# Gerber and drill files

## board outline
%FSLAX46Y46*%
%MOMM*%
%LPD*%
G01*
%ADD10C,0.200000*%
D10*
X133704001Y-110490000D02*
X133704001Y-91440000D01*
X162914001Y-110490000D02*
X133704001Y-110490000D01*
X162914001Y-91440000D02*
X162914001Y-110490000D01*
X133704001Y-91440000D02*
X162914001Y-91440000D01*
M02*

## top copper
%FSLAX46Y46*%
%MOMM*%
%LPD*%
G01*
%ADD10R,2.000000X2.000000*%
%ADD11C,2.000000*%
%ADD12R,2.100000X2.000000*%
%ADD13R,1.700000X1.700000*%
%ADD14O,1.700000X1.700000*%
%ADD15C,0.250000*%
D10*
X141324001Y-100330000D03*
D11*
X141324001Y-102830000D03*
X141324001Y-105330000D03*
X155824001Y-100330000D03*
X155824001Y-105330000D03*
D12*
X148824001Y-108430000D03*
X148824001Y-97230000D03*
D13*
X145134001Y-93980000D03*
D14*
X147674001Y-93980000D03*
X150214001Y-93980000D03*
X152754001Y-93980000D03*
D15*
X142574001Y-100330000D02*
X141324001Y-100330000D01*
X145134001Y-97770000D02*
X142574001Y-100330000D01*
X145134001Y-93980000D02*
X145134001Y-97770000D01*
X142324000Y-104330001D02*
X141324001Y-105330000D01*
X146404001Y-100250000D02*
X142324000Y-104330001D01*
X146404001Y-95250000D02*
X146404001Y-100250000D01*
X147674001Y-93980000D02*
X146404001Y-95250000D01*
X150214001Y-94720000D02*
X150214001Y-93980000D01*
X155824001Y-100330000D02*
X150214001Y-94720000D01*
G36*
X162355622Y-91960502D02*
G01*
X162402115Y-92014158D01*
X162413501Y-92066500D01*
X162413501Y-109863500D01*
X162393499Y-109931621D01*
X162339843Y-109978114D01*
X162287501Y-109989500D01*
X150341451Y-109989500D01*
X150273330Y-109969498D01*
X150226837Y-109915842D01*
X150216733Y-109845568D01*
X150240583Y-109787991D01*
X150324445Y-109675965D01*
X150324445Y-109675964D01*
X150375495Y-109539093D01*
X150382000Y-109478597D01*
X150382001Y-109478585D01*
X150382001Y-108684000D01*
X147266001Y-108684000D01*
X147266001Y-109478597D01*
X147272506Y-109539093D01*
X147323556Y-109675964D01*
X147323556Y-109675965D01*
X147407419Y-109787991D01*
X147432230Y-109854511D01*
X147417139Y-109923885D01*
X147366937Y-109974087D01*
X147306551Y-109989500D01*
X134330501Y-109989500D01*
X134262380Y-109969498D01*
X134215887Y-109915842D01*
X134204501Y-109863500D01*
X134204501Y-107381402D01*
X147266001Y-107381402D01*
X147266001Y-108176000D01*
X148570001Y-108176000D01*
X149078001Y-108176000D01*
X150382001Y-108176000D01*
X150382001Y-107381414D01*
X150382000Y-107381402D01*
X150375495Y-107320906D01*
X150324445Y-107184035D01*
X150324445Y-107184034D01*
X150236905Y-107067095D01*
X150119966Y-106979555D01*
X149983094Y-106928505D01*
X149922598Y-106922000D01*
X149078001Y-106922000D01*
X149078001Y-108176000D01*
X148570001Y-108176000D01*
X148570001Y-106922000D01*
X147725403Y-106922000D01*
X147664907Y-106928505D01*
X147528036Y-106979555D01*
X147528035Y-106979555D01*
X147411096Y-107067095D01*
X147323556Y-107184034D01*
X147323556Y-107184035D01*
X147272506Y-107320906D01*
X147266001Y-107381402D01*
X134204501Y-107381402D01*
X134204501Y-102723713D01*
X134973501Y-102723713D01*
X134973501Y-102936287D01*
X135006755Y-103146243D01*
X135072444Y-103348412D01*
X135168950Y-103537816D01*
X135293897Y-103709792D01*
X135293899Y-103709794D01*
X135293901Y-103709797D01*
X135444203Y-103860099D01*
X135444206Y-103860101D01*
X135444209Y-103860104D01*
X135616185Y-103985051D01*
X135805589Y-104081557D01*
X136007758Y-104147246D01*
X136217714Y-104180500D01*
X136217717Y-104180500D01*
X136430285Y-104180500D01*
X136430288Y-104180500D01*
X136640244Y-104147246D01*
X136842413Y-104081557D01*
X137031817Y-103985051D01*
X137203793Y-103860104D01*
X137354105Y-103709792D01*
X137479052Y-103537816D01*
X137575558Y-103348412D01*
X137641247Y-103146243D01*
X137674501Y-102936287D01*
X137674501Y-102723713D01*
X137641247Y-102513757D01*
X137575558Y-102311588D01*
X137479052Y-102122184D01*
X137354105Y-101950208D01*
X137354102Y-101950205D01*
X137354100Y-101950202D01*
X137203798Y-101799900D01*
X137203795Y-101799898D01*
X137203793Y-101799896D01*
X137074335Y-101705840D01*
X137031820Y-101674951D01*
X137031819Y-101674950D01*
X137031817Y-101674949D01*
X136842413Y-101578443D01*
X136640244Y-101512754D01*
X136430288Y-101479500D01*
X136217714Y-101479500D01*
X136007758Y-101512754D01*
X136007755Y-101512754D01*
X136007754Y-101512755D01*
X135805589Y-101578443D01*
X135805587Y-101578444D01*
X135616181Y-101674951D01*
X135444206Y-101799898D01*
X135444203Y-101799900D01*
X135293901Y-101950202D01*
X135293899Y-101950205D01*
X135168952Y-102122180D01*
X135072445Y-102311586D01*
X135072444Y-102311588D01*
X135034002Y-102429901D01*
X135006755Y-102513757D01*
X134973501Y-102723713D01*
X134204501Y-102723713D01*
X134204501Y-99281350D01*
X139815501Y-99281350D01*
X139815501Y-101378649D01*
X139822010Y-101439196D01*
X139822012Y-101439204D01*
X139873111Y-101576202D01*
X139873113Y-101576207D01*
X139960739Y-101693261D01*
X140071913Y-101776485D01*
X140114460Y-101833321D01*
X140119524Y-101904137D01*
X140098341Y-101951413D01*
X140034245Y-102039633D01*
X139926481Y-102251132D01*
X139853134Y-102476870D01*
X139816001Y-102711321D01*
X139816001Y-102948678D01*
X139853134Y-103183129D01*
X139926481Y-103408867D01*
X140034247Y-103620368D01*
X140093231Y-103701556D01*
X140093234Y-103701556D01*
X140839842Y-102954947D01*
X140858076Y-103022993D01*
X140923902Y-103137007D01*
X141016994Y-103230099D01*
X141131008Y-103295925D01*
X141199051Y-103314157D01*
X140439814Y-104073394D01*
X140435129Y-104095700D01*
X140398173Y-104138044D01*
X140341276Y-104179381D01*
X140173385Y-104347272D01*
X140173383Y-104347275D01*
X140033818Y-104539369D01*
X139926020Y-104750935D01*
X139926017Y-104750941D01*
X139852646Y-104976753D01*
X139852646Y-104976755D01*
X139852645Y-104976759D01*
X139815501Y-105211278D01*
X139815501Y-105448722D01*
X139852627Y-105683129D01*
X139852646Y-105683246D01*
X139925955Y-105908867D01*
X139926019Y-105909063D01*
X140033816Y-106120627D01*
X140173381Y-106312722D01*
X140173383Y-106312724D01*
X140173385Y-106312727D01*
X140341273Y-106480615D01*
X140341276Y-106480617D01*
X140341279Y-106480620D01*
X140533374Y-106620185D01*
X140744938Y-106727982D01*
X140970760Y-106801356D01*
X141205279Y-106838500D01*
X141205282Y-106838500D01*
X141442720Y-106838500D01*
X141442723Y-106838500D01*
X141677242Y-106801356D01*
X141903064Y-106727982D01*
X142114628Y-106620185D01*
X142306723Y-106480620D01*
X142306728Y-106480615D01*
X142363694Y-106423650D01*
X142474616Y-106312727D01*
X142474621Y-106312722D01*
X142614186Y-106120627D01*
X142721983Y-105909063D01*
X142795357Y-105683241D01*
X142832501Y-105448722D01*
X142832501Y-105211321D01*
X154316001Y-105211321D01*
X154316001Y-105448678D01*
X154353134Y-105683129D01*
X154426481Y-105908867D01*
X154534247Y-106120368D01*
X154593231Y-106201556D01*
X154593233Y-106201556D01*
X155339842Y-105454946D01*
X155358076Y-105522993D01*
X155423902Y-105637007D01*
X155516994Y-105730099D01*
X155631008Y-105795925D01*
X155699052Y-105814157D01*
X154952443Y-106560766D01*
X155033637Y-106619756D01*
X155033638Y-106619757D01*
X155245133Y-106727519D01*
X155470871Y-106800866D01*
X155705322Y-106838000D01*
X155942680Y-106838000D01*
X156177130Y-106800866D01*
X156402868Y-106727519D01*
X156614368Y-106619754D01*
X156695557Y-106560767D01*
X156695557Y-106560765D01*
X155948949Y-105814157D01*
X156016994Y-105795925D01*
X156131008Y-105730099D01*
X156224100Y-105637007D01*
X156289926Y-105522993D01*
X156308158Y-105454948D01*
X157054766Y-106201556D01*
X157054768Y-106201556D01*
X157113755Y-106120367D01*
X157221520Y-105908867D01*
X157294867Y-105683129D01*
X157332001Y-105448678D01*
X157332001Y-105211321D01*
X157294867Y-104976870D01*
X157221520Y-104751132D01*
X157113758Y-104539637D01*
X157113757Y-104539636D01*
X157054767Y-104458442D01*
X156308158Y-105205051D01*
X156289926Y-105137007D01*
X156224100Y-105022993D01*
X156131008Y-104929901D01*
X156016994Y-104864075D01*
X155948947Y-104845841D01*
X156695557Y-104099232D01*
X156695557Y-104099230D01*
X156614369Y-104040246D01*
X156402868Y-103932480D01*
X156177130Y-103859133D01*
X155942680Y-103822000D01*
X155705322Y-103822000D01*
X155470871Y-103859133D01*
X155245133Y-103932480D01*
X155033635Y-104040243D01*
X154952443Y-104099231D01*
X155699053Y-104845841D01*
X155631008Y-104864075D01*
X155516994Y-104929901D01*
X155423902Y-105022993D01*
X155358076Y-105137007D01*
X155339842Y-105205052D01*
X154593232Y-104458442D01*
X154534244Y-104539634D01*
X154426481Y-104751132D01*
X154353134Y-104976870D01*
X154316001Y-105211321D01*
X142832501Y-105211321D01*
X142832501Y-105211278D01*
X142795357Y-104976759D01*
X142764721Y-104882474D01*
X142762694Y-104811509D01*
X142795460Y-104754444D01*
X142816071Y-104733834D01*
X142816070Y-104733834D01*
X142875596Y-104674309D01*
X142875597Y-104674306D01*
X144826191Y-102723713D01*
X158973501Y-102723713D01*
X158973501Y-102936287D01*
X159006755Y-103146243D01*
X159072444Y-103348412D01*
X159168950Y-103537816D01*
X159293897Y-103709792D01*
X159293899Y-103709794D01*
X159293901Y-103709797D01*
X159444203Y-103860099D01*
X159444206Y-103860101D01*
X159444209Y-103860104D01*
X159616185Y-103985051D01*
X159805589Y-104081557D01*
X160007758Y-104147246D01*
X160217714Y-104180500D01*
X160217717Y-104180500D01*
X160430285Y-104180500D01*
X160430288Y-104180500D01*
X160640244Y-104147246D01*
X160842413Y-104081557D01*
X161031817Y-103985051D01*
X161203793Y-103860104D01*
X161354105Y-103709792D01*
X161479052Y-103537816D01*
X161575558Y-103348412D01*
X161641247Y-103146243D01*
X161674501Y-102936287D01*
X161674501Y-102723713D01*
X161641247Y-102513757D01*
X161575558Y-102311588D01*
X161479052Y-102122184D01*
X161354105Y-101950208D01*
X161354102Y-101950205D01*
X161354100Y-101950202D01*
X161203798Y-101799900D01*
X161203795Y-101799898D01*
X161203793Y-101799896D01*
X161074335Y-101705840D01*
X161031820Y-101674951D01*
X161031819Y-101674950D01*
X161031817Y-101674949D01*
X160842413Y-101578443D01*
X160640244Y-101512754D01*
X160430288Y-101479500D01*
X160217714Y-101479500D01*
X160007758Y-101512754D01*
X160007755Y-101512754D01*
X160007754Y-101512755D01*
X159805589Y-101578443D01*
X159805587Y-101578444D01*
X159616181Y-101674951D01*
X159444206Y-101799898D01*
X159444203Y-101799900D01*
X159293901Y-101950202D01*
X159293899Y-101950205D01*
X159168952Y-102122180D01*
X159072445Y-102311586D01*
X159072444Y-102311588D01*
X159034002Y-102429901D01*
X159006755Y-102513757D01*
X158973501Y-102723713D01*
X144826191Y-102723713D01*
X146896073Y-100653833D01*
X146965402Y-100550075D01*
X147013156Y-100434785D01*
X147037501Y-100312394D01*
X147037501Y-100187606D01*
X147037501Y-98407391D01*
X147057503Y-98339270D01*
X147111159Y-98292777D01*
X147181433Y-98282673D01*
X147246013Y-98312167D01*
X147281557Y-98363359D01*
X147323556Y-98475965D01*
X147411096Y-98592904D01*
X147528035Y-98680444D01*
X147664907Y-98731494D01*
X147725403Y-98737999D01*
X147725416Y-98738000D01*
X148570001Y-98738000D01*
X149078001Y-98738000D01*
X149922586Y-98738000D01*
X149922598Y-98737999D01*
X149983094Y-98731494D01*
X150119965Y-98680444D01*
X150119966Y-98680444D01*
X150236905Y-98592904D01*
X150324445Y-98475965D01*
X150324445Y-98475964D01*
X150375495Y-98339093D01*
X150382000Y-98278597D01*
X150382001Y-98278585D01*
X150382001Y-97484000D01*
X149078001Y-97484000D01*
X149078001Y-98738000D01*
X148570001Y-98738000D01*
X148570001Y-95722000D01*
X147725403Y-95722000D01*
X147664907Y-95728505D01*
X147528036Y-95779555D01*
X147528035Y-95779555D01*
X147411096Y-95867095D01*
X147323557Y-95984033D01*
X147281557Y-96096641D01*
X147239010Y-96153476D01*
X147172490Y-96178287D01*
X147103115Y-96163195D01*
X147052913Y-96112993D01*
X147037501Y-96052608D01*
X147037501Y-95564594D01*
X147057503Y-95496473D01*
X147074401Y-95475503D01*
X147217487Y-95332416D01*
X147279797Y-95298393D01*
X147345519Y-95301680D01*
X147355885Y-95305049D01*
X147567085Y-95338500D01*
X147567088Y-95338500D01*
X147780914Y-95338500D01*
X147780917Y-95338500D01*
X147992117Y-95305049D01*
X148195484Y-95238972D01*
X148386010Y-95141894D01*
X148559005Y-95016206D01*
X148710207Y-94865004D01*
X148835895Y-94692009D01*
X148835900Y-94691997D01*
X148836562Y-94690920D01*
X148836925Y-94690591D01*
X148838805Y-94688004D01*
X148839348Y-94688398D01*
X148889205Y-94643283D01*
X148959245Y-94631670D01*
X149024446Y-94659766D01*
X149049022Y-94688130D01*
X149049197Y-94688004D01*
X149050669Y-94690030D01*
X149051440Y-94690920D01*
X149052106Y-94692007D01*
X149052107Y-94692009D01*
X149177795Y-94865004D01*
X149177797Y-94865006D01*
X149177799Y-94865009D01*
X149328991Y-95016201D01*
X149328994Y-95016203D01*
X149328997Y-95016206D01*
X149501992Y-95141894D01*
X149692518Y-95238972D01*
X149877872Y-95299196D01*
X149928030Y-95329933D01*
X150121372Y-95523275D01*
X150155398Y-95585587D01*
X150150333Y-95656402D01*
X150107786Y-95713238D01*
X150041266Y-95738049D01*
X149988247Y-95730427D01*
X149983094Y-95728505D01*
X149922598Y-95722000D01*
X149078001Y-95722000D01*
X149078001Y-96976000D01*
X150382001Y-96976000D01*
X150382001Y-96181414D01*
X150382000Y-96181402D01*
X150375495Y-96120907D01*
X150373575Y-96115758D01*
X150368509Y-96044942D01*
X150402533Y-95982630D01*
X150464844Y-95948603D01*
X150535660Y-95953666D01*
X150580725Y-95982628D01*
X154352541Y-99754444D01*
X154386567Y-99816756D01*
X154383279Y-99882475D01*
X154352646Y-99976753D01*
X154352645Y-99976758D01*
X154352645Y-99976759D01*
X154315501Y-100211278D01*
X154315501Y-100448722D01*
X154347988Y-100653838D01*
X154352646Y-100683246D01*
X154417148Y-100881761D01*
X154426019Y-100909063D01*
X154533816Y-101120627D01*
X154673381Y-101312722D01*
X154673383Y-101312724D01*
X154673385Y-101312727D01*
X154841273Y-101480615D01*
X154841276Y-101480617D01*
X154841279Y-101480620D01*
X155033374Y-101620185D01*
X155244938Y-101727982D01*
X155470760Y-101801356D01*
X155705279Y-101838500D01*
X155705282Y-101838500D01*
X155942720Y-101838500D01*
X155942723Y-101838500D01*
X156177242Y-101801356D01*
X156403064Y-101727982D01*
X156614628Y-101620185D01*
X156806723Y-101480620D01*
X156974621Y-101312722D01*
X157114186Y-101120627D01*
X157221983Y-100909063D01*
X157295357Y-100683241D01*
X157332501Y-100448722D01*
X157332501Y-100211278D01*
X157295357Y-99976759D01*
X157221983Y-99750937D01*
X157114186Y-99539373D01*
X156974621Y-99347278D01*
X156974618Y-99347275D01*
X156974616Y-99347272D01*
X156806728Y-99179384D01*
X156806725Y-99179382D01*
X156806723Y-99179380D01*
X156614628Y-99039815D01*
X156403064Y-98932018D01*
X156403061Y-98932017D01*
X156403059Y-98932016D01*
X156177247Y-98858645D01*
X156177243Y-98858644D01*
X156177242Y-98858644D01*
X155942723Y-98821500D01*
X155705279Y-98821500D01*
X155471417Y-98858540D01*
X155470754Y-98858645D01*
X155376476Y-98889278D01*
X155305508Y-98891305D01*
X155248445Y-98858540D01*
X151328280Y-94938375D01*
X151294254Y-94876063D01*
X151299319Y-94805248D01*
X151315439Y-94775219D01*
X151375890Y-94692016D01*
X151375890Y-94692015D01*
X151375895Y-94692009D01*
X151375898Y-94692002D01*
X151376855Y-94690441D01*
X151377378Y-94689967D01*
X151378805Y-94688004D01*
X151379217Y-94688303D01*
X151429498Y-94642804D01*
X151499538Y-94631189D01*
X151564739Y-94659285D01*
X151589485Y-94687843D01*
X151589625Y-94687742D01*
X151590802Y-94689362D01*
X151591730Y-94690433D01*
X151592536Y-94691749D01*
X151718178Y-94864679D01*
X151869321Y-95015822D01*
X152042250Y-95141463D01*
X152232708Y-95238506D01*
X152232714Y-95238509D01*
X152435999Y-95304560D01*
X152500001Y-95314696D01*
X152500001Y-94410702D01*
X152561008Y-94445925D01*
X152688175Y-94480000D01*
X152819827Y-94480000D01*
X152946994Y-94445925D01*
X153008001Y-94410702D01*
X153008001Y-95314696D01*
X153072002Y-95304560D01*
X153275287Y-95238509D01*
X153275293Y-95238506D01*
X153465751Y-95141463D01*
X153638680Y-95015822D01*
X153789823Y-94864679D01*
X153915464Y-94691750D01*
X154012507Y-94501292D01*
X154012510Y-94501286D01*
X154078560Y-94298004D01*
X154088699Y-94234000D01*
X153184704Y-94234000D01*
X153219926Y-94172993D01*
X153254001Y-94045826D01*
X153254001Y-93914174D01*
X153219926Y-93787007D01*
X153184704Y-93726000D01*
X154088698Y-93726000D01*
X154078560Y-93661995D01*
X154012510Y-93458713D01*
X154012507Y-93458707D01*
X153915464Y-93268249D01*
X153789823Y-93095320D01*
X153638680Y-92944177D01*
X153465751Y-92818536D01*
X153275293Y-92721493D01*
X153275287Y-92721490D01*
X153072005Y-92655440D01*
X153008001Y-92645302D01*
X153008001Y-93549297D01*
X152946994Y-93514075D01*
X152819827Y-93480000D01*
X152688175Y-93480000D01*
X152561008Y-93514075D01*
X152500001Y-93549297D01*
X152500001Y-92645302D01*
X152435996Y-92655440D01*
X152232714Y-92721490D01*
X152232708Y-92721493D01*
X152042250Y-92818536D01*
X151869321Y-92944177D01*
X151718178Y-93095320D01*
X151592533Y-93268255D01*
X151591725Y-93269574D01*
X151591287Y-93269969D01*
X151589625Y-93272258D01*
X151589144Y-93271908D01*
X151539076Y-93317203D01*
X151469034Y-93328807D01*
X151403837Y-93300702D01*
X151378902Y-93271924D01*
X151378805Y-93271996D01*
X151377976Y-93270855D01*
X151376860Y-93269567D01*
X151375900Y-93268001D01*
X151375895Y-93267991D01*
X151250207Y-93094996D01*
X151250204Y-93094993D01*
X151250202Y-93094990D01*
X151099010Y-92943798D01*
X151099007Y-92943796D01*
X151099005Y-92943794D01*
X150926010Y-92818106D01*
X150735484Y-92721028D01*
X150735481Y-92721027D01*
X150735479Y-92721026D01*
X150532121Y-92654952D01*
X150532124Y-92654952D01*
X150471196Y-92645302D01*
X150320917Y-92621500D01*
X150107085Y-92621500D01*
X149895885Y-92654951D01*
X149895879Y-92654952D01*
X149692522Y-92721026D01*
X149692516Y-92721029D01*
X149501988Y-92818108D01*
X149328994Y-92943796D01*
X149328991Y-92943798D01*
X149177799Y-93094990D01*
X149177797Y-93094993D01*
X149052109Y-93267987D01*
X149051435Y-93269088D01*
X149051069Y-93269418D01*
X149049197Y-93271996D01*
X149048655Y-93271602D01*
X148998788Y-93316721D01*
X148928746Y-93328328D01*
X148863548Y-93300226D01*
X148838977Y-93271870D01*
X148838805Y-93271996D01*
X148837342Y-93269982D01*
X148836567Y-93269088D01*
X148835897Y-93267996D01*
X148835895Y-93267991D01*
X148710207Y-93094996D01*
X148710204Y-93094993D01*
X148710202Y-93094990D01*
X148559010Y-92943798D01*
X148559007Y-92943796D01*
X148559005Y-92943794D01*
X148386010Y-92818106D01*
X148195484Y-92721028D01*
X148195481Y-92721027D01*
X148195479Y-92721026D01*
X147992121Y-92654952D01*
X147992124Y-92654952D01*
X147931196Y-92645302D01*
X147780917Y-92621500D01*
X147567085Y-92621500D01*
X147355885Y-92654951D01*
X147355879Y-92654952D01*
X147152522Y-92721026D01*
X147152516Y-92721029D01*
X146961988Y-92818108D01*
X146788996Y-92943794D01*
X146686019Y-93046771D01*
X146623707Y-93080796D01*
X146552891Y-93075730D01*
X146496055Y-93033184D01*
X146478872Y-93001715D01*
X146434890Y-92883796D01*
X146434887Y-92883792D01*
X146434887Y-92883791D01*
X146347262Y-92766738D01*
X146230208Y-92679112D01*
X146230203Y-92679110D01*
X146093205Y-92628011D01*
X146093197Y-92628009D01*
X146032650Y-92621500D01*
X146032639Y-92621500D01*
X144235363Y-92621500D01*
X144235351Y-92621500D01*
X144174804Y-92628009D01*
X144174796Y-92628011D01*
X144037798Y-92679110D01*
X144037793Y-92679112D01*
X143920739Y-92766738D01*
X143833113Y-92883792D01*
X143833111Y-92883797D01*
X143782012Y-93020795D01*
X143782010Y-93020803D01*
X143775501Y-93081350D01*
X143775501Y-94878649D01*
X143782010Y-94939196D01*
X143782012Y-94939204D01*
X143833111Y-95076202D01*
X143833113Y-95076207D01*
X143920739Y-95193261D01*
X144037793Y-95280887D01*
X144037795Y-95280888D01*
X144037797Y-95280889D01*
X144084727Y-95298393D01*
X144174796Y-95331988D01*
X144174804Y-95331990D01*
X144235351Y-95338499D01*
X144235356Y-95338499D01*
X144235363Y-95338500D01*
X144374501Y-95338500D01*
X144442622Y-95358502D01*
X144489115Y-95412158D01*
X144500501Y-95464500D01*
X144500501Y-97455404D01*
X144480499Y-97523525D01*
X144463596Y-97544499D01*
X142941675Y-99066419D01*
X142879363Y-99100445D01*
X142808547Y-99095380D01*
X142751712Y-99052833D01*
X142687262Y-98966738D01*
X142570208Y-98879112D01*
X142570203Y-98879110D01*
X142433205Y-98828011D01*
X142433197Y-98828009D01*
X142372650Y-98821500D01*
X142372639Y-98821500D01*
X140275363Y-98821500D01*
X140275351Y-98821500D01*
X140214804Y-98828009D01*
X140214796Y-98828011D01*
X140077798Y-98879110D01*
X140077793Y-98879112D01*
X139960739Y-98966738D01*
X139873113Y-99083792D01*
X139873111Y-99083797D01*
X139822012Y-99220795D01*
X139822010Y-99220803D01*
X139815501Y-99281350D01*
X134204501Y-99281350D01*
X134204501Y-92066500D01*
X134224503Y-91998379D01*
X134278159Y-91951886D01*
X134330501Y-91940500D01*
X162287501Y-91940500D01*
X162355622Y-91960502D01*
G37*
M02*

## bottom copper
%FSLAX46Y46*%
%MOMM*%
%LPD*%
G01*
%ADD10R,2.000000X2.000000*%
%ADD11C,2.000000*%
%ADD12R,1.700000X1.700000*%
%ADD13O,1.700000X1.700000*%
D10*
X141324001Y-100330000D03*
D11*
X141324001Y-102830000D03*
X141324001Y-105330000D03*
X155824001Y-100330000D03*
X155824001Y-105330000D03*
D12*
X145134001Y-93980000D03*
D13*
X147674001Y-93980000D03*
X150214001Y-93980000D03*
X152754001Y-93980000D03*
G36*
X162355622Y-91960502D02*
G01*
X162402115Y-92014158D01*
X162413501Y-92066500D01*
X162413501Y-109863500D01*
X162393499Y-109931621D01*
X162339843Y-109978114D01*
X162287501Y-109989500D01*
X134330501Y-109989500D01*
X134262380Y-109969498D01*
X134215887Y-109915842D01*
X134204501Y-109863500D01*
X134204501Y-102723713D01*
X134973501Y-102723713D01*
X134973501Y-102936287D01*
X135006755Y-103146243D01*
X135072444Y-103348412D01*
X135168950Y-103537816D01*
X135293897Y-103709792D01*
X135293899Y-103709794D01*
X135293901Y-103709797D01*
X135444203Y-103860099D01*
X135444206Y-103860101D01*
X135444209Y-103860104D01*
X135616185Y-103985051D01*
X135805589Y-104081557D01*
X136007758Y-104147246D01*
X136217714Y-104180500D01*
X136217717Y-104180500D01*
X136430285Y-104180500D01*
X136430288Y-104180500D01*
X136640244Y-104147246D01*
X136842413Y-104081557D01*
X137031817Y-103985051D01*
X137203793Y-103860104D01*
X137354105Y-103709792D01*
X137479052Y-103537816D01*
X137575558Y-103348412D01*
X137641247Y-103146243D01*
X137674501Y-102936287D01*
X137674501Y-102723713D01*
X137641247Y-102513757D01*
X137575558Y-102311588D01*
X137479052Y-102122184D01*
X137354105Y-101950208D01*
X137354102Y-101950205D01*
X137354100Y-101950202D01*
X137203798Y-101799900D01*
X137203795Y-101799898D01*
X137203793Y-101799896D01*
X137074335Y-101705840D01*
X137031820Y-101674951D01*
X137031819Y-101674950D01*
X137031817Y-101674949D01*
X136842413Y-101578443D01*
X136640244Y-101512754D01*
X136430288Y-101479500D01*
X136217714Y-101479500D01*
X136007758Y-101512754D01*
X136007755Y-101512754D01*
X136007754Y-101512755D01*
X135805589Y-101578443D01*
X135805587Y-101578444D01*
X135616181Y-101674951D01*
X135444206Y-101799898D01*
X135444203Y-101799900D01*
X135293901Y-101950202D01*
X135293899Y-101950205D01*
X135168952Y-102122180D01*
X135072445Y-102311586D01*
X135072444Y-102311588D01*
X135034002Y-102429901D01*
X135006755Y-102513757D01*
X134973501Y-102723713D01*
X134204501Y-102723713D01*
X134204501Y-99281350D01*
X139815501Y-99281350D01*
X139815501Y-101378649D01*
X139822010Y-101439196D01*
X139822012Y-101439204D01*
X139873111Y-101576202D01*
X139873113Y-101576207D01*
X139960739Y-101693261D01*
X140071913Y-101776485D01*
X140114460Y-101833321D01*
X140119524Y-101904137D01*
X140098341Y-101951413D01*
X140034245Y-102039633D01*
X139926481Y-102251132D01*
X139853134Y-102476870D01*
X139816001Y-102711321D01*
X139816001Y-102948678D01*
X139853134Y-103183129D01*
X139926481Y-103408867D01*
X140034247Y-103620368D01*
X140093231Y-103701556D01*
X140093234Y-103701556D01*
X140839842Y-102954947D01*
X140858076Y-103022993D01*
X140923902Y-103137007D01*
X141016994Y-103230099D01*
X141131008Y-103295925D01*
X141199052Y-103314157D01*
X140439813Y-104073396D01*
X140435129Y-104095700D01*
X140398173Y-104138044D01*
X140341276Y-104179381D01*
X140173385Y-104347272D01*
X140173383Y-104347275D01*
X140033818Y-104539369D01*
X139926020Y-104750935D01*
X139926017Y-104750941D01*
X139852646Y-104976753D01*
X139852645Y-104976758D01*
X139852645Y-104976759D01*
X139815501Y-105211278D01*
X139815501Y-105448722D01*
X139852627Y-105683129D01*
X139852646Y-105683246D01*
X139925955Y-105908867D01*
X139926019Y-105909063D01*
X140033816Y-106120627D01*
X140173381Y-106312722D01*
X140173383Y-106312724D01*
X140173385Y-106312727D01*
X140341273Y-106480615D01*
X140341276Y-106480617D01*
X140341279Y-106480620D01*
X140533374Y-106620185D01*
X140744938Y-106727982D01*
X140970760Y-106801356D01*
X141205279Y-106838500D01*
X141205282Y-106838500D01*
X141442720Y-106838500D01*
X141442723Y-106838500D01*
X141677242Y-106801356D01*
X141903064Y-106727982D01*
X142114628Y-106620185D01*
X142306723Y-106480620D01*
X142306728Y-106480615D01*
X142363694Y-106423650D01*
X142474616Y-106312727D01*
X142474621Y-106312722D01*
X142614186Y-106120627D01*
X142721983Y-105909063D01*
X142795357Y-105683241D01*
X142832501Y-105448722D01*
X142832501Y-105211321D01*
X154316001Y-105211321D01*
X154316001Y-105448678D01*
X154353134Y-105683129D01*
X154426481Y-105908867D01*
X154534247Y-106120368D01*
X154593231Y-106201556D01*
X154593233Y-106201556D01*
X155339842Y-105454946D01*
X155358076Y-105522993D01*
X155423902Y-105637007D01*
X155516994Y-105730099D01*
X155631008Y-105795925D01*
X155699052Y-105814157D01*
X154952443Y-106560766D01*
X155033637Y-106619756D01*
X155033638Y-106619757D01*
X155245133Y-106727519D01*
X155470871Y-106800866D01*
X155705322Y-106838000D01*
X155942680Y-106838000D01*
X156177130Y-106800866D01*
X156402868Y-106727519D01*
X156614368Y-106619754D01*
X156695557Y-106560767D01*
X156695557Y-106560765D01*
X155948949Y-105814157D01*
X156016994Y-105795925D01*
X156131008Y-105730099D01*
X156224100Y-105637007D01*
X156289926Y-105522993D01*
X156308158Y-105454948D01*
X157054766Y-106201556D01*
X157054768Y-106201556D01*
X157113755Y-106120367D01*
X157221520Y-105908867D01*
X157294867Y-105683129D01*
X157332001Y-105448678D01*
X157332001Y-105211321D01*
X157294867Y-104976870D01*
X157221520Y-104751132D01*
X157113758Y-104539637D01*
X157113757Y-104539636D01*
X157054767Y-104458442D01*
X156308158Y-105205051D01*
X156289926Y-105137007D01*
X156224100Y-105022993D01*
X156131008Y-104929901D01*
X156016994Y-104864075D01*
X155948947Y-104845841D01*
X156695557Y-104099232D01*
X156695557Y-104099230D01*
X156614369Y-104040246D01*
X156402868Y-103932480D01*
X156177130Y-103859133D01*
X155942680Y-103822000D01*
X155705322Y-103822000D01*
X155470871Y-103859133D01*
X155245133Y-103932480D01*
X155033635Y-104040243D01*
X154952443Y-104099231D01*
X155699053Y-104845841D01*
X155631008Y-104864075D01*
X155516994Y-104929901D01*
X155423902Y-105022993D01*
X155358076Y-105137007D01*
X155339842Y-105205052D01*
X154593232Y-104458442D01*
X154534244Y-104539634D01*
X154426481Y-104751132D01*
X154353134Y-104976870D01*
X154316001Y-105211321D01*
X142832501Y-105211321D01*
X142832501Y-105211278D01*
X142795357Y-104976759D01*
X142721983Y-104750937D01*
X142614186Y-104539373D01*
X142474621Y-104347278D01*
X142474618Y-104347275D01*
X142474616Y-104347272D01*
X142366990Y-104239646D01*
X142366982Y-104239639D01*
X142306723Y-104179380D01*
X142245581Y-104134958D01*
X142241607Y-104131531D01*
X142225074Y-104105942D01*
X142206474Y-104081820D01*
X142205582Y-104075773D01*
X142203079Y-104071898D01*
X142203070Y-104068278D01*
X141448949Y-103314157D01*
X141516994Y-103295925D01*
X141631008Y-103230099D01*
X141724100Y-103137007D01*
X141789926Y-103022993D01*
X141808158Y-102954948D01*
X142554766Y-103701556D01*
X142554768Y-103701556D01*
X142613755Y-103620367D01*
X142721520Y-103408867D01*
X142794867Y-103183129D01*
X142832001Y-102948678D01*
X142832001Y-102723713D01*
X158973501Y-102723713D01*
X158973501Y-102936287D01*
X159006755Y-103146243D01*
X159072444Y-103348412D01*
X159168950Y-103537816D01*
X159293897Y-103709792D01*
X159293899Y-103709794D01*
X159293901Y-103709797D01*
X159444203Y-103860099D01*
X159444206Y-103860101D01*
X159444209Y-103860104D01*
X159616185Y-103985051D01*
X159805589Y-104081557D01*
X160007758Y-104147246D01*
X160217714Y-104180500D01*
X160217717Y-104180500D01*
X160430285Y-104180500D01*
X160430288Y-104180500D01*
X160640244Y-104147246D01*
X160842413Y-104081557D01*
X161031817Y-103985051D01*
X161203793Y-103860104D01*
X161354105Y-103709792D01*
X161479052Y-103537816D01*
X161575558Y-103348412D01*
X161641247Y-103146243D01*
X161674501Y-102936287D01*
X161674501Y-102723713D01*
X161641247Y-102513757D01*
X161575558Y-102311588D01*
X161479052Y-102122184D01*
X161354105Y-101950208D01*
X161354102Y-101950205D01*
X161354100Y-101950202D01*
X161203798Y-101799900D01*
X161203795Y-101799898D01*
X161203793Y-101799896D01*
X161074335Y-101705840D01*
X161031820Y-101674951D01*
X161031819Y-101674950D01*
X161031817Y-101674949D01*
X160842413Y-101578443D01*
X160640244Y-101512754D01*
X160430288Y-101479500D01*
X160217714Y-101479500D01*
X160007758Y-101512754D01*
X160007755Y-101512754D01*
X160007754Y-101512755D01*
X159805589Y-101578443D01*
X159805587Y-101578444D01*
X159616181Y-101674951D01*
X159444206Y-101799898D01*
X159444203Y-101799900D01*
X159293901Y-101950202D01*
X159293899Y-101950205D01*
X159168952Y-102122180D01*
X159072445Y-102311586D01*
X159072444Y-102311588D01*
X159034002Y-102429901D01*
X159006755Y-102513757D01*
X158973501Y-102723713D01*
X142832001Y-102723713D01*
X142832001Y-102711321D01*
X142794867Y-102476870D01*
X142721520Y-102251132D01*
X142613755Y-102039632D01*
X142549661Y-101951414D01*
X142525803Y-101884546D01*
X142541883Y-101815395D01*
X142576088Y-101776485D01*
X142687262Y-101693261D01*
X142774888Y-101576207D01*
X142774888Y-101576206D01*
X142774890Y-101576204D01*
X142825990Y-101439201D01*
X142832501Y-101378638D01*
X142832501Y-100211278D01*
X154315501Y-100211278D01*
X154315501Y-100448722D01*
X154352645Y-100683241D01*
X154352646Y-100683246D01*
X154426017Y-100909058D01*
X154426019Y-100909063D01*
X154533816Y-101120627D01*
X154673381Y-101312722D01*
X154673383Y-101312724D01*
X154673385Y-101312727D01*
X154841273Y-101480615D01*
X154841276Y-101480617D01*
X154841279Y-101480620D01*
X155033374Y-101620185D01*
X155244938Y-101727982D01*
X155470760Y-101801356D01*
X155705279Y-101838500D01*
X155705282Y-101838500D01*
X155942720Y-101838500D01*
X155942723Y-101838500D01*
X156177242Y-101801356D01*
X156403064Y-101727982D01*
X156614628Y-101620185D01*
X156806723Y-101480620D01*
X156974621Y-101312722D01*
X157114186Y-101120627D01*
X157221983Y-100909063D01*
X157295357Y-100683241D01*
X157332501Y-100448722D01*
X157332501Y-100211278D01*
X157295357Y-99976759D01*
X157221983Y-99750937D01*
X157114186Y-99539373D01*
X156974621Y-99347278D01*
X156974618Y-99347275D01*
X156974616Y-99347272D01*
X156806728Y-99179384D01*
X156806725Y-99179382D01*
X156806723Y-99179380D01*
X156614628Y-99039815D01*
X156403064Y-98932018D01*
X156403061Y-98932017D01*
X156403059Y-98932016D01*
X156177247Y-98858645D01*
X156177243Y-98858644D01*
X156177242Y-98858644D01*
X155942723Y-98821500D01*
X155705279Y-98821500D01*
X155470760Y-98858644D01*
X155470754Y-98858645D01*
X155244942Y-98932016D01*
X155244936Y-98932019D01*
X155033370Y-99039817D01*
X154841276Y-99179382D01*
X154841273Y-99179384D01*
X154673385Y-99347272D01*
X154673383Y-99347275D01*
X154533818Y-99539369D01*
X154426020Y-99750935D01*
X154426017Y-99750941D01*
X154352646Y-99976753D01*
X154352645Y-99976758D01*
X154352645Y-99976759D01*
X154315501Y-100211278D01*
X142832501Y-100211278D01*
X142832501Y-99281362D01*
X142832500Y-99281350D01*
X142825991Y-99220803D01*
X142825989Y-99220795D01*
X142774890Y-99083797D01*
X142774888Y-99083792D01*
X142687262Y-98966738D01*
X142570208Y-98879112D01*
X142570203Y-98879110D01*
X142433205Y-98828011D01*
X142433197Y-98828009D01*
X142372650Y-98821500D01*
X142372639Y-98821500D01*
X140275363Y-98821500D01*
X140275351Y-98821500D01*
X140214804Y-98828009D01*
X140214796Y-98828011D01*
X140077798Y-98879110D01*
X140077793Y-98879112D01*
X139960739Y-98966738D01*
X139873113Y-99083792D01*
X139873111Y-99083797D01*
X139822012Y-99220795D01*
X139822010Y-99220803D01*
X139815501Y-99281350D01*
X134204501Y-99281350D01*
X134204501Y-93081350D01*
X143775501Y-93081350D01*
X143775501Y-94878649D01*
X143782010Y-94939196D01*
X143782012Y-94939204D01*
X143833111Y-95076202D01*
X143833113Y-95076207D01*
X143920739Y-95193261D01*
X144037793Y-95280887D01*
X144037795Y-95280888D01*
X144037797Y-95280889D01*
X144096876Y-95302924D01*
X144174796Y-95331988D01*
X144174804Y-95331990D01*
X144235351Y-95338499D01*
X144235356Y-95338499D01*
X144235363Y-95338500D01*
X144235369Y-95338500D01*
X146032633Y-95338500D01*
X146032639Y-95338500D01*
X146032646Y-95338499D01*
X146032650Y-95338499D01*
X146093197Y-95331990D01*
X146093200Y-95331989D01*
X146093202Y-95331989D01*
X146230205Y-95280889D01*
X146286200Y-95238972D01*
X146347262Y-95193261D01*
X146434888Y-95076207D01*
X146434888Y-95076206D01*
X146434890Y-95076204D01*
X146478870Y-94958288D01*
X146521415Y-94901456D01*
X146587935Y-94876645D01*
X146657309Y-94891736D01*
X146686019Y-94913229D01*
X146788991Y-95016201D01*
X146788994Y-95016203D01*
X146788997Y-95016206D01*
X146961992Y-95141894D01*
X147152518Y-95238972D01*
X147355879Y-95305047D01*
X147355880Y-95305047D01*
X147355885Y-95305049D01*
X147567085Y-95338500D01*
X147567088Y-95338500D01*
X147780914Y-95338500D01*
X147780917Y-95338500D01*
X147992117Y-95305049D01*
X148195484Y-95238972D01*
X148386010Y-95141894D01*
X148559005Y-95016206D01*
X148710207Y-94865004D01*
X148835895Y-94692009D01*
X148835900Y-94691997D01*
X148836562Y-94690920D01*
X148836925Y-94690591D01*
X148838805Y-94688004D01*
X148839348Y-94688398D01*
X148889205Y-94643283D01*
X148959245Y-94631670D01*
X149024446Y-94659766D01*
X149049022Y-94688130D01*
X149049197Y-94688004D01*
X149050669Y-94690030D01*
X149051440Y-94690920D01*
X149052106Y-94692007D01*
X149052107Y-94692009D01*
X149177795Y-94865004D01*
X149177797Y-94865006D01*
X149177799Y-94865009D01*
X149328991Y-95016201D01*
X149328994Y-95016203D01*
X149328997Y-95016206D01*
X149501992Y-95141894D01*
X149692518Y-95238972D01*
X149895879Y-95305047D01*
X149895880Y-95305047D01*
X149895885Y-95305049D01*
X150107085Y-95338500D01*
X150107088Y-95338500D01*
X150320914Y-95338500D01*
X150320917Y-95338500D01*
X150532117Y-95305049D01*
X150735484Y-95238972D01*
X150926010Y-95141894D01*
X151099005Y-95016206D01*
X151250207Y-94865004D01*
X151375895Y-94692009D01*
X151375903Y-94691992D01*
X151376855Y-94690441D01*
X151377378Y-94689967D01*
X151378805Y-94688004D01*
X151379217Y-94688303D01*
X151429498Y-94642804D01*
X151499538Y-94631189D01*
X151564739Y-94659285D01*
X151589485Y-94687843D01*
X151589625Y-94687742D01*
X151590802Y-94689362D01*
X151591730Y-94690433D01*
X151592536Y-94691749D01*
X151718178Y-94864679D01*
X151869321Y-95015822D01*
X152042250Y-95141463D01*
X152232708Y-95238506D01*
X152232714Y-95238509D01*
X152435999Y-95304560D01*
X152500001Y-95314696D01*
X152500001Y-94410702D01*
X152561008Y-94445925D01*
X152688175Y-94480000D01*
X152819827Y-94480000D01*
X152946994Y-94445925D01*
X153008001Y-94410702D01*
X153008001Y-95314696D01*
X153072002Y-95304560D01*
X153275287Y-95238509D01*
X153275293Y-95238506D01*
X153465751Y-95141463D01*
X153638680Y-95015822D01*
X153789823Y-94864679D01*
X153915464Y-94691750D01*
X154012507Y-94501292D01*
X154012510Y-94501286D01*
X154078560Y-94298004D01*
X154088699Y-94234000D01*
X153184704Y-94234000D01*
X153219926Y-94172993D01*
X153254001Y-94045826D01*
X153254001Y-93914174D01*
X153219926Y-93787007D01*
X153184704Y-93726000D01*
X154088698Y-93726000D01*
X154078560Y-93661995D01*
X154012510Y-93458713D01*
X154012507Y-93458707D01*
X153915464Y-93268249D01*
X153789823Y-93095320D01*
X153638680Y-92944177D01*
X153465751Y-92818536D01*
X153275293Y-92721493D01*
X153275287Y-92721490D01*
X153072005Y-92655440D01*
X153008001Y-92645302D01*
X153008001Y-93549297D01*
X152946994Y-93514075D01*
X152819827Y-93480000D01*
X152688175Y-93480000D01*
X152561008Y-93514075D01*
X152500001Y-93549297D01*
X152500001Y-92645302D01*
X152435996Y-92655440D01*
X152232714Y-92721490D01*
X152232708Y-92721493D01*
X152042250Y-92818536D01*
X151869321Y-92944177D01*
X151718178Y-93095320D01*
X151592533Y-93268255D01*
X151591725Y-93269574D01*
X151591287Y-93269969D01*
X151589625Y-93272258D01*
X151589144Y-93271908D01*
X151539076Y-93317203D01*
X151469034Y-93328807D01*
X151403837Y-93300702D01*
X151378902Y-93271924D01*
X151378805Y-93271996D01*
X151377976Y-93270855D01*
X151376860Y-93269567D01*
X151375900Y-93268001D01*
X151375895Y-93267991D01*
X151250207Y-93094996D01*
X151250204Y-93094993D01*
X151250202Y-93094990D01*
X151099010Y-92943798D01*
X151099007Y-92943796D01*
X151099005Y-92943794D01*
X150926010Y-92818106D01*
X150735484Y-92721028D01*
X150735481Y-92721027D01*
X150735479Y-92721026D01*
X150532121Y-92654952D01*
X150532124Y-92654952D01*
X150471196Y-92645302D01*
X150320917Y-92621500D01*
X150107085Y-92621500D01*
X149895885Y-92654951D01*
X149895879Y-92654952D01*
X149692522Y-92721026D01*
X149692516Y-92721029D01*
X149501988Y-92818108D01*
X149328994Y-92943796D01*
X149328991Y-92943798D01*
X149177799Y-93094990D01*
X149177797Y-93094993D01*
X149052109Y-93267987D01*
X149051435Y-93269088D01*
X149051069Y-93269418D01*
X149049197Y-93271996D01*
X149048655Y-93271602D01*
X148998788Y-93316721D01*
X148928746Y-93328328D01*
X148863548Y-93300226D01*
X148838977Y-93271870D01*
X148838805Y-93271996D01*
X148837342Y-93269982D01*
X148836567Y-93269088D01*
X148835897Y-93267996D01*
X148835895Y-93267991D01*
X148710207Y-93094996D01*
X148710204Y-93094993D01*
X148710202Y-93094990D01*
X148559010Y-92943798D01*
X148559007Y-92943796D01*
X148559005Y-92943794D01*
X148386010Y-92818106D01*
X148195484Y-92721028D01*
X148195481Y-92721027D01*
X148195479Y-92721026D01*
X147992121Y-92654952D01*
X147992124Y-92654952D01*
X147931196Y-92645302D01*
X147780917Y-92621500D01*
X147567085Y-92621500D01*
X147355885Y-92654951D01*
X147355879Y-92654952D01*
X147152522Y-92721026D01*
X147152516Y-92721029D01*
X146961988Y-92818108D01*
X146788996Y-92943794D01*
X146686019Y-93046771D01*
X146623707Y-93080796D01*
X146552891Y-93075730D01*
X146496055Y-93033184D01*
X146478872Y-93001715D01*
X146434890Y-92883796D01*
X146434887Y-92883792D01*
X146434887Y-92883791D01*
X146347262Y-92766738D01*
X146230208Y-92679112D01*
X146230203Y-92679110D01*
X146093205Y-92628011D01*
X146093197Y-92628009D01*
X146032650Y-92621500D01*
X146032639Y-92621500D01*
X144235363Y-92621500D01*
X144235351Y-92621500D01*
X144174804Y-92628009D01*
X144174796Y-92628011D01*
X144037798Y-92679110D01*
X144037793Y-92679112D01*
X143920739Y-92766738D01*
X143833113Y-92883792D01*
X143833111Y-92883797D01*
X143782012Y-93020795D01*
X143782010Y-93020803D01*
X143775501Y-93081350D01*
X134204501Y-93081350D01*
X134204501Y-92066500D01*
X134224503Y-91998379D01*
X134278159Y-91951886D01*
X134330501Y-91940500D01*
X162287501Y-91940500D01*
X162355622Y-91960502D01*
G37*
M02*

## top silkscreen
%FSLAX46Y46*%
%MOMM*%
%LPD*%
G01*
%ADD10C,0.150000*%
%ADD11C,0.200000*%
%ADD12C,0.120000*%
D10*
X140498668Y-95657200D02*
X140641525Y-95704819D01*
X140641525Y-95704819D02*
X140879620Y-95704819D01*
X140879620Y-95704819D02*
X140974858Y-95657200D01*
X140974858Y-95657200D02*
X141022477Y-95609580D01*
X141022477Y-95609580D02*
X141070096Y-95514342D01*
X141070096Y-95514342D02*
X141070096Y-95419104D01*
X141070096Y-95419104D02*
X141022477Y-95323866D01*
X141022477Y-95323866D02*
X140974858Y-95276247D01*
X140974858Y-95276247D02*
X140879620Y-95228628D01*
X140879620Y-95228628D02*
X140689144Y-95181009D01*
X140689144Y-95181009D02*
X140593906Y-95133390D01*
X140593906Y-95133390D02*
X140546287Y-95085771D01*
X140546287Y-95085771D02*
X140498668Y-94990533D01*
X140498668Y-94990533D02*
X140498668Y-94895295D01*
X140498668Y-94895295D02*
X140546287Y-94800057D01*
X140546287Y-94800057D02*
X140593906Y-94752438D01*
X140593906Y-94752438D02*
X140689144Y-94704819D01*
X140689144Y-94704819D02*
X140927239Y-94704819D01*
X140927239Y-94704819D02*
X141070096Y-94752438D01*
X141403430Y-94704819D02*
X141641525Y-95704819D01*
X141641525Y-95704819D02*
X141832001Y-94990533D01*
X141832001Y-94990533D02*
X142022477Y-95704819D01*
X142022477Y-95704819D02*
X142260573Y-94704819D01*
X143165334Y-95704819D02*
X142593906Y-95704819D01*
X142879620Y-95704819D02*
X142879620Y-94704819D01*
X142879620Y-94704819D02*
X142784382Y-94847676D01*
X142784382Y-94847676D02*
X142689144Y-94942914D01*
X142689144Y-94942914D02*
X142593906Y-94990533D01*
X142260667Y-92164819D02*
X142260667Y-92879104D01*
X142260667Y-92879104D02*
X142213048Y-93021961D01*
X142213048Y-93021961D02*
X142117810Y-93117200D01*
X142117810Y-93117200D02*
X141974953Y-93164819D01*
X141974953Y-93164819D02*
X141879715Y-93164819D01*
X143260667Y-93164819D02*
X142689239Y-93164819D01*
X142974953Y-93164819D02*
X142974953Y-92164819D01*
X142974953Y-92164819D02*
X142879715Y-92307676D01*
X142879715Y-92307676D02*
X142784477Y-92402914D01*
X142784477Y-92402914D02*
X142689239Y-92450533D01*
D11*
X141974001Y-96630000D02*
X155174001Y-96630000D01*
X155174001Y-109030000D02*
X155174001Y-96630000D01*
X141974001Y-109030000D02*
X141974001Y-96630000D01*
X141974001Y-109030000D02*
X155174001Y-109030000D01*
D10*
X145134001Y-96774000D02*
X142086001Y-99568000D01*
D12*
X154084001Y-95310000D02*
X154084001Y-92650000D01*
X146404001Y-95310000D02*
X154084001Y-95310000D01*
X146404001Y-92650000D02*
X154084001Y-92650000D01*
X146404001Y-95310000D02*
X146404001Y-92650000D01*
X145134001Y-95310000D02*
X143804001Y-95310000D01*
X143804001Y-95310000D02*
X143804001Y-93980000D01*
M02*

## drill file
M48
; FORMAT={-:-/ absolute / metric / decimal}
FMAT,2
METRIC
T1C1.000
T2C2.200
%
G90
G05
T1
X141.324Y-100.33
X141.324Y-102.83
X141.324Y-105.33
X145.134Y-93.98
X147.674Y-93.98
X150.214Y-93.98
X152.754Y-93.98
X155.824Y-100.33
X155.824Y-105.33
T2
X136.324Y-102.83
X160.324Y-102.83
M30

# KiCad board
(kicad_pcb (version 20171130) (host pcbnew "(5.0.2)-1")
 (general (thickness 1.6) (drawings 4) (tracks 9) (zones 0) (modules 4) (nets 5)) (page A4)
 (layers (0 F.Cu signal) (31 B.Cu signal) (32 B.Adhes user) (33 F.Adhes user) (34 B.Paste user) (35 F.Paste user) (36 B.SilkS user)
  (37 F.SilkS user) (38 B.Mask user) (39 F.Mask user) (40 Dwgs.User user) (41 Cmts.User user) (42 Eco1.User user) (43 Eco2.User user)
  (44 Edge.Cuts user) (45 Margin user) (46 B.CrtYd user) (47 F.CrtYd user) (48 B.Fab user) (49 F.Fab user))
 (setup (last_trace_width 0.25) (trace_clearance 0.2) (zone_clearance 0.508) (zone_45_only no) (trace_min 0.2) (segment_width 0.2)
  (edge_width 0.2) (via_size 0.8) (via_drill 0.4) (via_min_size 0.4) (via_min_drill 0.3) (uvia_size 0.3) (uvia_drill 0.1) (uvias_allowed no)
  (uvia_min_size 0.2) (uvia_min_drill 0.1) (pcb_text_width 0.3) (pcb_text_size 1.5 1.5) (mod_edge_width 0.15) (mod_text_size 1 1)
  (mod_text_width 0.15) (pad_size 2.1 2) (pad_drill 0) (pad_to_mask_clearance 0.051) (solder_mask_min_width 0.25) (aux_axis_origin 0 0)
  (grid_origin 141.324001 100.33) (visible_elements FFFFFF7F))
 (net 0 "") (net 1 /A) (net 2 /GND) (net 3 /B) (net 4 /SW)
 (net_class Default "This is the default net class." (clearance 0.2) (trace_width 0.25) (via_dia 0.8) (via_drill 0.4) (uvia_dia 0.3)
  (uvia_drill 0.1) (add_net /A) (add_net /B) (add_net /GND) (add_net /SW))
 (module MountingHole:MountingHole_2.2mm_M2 (layer F.Cu) (at 136.324001 102.83)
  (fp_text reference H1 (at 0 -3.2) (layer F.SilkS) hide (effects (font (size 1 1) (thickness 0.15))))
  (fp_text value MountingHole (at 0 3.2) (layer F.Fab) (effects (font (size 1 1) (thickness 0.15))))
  (pad 1 np_thru_hole circle (at 0 0) (size 2.2 2.2) (drill 2.2) (layers *.Cu *.Mask)))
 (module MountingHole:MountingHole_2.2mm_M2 (layer F.Cu) (at 160.324001 102.83)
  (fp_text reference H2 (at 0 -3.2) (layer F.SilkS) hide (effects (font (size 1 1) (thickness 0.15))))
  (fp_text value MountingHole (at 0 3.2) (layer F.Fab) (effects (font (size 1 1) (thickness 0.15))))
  (pad 1 np_thru_hole circle (at 0 0) (size 2.2 2.2) (drill 2.2) (layers *.Cu *.Mask)))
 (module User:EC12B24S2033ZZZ (layer F.Cu) (at 141.324001 100.33)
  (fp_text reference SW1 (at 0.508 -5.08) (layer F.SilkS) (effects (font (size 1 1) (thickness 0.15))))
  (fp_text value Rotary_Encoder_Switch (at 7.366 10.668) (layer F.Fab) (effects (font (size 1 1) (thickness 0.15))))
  (fp_line (start 0.65 -3.7) (end 13.85 -3.7) (layer F.SilkS) (width 0.2))
  (fp_line (start 13.85 8.7) (end 13.85 -3.7) (layer F.SilkS) (width 0.2))
  (fp_line (start 0.65 8.7) (end 0.65 -3.7) (layer F.SilkS) (width 0.2))
  (fp_line (start 0.65 8.7) (end 13.85 8.7) (layer F.SilkS) (width 0.2))
  (fp_line (start 3.81 -3.556) (end 0.762 -0.762) (layer F.SilkS) (width 0.15))
  (pad A thru_hole rect (at 0 0) (size 2 2) (drill 1) (layers *.Cu *.Mask) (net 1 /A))
  (pad C thru_hole circle (at 0 2.5) (size 2 2) (drill 1) (layers *.Cu *.Mask) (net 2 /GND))
  (pad B thru_hole circle (at 0 5) (size 2 2) (drill 1) (layers *.Cu *.Mask) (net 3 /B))
  (pad S1 thru_hole circle (at 14.5 0) (size 2 2) (drill 1) (layers *.Cu *.Mask) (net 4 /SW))
  (pad S2 thru_hole circle (at 14.5 5) (size 2 2) (drill 1) (layers *.Cu *.Mask) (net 2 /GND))
  (pad "" smd rect (at 7.5 8.1) (size 2.1 2) (layers F.Cu F.Paste F.Mask) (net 2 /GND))
  (pad "" smd rect (at 7.5 -3.1) (size 2.1 2) (layers F.Cu F.Paste F.Mask) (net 2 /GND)))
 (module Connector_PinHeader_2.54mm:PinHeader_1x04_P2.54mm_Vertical (layer F.Cu) (at 145.134001 93.98 90)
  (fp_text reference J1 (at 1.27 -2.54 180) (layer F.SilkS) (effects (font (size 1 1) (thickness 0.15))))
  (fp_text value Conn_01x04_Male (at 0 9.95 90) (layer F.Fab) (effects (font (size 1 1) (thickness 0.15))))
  (fp_line (start -1.33 8.95) (end 1.33 8.95) (layer F.SilkS) (width 0.12))
  (fp_line (start -1.33 1.27) (end -1.33 8.95) (layer F.SilkS) (width 0.12))
  (fp_line (start 1.33 1.27) (end 1.33 8.95) (layer F.SilkS) (width 0.12))
  (fp_line (start -1.33 1.27) (end 1.33 1.27) (layer F.SilkS) (width 0.12))
  (fp_line (start -1.33 0) (end -1.33 -1.33) (layer F.SilkS) (width 0.12))
  (fp_line (start -1.33 -1.33) (end 0 -1.33) (layer F.SilkS) (width 0.12))
  (pad 1 thru_hole rect (at 0 0 90) (size 1.7 1.7) (drill 1) (layers *.Cu *.Mask) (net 1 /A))
  (pad 2 thru_hole oval (at 0 2.54 90) (size 1.7 1.7) (drill 1) (layers *.Cu *.Mask) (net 3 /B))
  (pad 3 thru_hole oval (at 0 5.08 90) (size 1.7 1.7) (drill 1) (layers *.Cu *.Mask) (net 4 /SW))
  (pad 4 thru_hole oval (at 0 7.62 90) (size 1.7 1.7) (drill 1) (layers *.Cu *.Mask) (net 2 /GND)))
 (gr_line (start 133.704001 110.49) (end 133.704001 91.44) (layer Edge.Cuts) (width 0.2))
 (gr_line (start 162.914001 110.49) (end 133.704001 110.49) (layer Edge.Cuts) (width 0.2))
 (gr_line (start 162.914001 91.44) (end 162.914001 110.49) (layer Edge.Cuts) (width 0.2))
 (gr_line (start 133.704001 91.44) (end 162.914001 91.44) (layer Edge.Cuts) (width 0.2))
 (segment (start 142.574001 100.33) (end 141.324001 100.33) (width 0.25) (layer F.Cu) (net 1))
 (segment (start 145.134001 97.77) (end 142.574001 100.33) (width 0.25) (layer F.Cu) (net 1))
 (segment (start 145.134001 93.98) (end 145.134001 97.77) (width 0.25) (layer F.Cu) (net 1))
 (segment (start 142.324 104.330001) (end 141.324001 105.33) (width 0.25) (layer F.Cu) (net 3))
 (segment (start 146.404001 100.25) (end 142.324 104.330001) (width 0.25) (layer F.Cu) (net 3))
 (segment (start 146.404001 95.25) (end 146.404001 100.25) (width 0.25) (layer F.Cu) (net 3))
 (segment (start 147.674001 93.98) (end 146.404001 95.25) (width 0.25) (layer F.Cu) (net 3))
 (segment (start 150.214001 94.72) (end 150.214001 93.98) (width 0.25) (layer F.Cu) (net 4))
 (segment (start 155.824001 100.33) (end 150.214001 94.72) (width 0.25) (layer F.Cu) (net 4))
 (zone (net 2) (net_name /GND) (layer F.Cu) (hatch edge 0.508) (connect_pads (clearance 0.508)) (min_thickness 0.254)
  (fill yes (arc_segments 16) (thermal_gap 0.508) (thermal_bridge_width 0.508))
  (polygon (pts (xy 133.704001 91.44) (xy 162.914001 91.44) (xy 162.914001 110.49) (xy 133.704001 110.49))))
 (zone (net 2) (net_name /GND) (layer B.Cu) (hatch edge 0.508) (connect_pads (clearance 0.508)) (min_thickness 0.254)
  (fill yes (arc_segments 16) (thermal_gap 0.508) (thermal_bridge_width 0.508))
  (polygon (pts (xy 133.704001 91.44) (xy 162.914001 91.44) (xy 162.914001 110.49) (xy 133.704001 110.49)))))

